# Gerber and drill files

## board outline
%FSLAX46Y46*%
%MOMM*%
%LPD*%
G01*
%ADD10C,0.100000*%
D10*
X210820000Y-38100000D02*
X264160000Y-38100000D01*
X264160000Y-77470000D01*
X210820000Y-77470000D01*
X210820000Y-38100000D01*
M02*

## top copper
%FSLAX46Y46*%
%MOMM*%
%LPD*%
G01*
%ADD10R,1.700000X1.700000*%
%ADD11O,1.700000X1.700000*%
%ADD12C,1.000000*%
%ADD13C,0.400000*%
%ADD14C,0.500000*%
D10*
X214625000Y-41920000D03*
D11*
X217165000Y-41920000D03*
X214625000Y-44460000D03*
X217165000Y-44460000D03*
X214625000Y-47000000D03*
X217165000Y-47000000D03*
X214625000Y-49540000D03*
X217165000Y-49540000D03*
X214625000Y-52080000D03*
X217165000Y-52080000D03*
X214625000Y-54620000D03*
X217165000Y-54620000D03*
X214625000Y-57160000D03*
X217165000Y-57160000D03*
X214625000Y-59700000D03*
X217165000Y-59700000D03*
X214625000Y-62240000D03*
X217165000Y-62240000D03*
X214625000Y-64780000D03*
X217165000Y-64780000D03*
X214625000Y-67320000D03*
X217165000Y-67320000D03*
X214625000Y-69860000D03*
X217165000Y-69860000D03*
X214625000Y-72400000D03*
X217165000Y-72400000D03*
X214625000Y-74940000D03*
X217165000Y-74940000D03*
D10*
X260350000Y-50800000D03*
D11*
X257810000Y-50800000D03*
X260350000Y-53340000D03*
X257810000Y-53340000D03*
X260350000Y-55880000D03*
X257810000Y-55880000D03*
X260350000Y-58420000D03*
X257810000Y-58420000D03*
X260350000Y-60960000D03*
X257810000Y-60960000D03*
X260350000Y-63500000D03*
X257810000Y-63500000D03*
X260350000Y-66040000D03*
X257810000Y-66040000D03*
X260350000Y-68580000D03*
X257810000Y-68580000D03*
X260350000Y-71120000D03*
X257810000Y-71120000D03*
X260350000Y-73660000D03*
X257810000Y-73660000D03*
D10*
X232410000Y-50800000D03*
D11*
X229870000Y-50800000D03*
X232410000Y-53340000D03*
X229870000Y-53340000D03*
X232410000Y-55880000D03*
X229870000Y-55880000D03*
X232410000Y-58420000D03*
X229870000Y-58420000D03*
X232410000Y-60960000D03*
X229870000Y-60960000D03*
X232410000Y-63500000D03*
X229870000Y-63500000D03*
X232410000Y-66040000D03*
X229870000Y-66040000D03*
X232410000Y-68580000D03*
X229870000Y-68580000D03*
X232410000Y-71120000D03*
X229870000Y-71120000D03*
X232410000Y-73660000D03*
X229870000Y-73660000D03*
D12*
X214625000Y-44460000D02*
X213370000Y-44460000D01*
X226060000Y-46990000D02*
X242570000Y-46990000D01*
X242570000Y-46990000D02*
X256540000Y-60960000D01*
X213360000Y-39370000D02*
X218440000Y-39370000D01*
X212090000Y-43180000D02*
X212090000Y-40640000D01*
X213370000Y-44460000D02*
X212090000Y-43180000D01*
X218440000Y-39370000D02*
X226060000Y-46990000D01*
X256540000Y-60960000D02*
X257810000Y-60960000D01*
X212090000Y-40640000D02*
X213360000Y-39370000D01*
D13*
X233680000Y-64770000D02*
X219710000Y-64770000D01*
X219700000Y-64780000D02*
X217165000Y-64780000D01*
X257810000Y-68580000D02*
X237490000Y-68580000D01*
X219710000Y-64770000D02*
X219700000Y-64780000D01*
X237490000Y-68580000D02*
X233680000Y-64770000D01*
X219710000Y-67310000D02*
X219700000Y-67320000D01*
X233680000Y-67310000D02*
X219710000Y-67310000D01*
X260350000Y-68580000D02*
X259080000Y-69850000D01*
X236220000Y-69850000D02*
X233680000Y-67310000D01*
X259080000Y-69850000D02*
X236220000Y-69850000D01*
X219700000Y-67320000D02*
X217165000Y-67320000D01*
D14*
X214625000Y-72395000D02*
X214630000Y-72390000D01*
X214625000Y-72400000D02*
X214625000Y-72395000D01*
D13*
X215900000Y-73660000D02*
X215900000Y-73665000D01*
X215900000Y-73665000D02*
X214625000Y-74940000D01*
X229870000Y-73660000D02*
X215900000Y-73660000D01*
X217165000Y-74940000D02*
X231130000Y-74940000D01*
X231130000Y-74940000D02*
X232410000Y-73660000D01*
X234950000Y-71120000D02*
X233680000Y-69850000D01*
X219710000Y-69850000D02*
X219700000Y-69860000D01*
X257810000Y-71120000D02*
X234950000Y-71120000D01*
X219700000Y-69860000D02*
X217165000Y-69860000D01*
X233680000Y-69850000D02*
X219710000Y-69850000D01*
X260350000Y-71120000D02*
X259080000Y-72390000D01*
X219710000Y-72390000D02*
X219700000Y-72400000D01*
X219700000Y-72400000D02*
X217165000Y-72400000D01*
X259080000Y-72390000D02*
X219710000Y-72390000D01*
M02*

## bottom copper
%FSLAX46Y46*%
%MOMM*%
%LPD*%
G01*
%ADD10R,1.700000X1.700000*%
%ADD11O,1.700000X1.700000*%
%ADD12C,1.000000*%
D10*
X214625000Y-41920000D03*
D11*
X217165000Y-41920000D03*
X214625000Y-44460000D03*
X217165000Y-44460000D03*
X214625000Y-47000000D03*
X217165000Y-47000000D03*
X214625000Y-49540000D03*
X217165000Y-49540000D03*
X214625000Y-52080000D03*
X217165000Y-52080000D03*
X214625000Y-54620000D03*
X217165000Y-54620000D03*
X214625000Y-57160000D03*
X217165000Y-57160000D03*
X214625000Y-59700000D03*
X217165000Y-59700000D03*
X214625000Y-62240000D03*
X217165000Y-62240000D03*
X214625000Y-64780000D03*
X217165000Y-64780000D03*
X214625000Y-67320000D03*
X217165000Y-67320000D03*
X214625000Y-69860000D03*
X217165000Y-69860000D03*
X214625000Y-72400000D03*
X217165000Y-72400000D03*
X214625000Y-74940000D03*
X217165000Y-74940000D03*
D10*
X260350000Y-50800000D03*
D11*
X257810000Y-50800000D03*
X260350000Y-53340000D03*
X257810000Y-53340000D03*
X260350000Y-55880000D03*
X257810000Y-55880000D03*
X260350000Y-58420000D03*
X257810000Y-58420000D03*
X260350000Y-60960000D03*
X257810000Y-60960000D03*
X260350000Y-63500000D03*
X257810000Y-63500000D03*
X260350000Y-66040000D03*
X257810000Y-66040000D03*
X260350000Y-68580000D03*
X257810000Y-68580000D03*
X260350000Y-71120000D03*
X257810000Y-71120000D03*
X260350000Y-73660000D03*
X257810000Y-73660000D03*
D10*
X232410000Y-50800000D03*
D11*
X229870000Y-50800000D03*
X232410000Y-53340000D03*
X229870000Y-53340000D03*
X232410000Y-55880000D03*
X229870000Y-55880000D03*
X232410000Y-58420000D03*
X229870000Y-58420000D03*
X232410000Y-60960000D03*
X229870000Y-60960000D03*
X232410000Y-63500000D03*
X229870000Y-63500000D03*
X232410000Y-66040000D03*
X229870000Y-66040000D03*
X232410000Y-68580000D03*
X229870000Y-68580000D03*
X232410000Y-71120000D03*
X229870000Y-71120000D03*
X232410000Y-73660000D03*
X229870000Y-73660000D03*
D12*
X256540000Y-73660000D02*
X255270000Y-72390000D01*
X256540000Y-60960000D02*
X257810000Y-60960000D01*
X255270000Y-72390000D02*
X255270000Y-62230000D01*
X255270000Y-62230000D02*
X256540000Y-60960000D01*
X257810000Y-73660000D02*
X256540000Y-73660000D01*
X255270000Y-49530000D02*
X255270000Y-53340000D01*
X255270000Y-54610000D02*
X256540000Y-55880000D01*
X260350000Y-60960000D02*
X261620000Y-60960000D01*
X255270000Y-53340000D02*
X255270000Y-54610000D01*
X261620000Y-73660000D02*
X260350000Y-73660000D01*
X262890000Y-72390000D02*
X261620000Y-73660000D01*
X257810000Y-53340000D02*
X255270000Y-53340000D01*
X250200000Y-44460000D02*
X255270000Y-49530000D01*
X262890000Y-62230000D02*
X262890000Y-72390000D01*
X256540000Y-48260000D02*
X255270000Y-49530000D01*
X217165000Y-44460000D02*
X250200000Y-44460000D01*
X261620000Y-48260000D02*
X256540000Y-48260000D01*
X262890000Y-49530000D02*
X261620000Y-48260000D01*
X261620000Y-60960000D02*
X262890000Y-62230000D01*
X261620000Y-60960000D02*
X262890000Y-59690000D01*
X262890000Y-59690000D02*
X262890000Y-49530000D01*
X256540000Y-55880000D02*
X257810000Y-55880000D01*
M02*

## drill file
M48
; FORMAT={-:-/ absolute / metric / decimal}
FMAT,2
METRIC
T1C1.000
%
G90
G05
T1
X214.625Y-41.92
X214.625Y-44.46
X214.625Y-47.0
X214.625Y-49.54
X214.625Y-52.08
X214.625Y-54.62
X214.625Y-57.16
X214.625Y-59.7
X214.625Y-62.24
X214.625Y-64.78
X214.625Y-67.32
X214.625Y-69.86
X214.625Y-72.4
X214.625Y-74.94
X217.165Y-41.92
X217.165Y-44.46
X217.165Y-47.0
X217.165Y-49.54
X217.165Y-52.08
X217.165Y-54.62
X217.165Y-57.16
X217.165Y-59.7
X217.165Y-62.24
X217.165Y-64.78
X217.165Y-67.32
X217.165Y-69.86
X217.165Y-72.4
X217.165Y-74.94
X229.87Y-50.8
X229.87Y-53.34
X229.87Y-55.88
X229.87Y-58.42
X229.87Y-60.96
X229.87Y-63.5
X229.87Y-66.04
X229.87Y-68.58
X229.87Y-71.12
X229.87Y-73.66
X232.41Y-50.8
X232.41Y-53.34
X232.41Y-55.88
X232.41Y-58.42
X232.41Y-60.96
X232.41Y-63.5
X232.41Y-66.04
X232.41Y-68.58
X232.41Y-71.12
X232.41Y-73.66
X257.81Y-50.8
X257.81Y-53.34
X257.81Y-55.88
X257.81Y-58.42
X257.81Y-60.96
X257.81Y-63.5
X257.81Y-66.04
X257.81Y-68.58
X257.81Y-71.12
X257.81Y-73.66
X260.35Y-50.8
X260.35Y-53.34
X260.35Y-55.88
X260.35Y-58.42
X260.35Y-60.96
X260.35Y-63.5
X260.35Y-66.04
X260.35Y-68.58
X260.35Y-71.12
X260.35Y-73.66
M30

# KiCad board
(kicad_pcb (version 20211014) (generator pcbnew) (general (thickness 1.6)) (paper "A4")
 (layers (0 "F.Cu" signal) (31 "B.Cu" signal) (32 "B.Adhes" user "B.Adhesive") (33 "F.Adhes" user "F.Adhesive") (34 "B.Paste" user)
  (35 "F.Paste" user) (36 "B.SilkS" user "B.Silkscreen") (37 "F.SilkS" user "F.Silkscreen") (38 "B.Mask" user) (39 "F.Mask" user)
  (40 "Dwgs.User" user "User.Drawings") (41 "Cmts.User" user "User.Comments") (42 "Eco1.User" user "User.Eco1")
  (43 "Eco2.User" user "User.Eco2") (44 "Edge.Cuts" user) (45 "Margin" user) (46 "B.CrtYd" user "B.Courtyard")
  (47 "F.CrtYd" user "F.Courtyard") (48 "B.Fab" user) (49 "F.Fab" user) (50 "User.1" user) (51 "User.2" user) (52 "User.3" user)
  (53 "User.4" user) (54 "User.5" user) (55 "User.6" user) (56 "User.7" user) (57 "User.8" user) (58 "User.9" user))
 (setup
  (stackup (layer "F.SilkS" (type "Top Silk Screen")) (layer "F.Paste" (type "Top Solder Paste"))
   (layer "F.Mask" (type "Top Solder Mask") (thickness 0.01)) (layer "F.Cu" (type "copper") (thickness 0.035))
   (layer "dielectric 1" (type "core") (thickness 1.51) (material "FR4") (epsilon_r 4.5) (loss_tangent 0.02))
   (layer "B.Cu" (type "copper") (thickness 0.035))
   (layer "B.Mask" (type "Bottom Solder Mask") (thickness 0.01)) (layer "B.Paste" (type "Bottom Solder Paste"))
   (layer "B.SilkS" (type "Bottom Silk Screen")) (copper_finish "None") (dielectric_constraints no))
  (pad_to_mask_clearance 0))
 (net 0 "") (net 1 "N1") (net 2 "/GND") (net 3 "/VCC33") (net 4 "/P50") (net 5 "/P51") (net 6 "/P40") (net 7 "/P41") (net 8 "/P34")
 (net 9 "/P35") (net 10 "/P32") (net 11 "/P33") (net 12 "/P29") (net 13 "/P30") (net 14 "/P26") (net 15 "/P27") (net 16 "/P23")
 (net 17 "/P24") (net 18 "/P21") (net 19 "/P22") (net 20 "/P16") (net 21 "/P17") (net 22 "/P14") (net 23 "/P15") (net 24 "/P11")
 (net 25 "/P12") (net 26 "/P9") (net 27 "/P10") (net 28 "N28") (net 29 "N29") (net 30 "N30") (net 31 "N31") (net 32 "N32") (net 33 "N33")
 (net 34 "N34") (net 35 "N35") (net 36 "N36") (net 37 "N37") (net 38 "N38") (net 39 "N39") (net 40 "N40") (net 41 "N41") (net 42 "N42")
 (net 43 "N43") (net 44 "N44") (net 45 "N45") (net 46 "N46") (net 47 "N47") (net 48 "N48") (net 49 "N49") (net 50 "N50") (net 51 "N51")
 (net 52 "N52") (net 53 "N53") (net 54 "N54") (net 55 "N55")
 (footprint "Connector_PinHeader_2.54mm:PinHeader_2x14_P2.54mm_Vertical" (layer "F.Cu") (at 214.625 41.92)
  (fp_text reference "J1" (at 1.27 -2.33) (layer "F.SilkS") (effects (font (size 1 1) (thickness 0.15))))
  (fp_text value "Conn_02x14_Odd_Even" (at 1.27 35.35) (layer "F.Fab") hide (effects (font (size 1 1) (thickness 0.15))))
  (pad "1" thru_hole rect locked (at 0 0) (size 1.7 1.7) (drill 1) (layers *.Cu *.Mask) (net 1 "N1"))
  (pad "2" thru_hole oval locked (at 2.54 0) (size 1.7 1.7) (drill 1) (layers *.Cu *.Mask) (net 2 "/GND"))
  (pad "3" thru_hole oval locked (at 0 2.54) (size 1.7 1.7) (drill 1) (layers *.Cu *.Mask) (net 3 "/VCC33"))
  (pad "4" thru_hole oval locked (at 2.54 2.54) (size 1.7 1.7) (drill 1) (layers *.Cu *.Mask) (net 2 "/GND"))
  (pad "5" thru_hole oval locked (at 0 5.08) (size 1.7 1.7) (drill 1) (layers *.Cu *.Mask) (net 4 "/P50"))
  (pad "6" thru_hole oval locked (at 2.54 5.08) (size 1.7 1.7) (drill 1) (layers *.Cu *.Mask) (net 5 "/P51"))
  (pad "7" thru_hole oval locked (at 0 7.62) (size 1.7 1.7) (drill 1) (layers *.Cu *.Mask) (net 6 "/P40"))
  (pad "8" thru_hole oval locked (at 2.54 7.62) (size 1.7 1.7) (drill 1) (layers *.Cu *.Mask) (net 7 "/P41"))
  (pad "9" thru_hole oval locked (at 0 10.16) (size 1.7 1.7) (drill 1) (layers *.Cu *.Mask) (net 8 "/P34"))
  (pad "10" thru_hole oval locked (at 2.54 10.16) (size 1.7 1.7) (drill 1) (layers *.Cu *.Mask) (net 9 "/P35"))
  (pad "11" thru_hole oval locked (at 0 12.7) (size 1.7 1.7) (drill 1) (layers *.Cu *.Mask) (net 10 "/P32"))
  (pad "12" thru_hole oval locked (at 2.54 12.7) (size 1.7 1.7) (drill 1) (layers *.Cu *.Mask) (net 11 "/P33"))
  (pad "13" thru_hole oval locked (at 0 15.24) (size 1.7 1.7) (drill 1) (layers *.Cu *.Mask) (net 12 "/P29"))
  (pad "14" thru_hole oval locked (at 2.54 15.24) (size 1.7 1.7) (drill 1) (layers *.Cu *.Mask) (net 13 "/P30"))
  (pad "15" thru_hole oval locked (at 0 17.78) (size 1.7 1.7) (drill 1) (layers *.Cu *.Mask) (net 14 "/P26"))
  (pad "16" thru_hole oval locked (at 2.54 17.78) (size 1.7 1.7) (drill 1) (layers *.Cu *.Mask) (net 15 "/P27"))
  (pad "17" thru_hole oval locked (at 0 20.32) (size 1.7 1.7) (drill 1) (layers *.Cu *.Mask) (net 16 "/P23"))
  (pad "18" thru_hole oval locked (at 2.54 20.32) (size 1.7 1.7) (drill 1) (layers *.Cu *.Mask) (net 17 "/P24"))
  (pad "19" thru_hole oval locked (at 0 22.86) (size 1.7 1.7) (drill 1) (layers *.Cu *.Mask) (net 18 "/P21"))
  (pad "20" thru_hole oval locked (at 2.54 22.86) (size 1.7 1.7) (drill 1) (layers *.Cu *.Mask) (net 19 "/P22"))
  (pad "21" thru_hole oval locked (at 0 25.4) (size 1.7 1.7) (drill 1) (layers *.Cu *.Mask) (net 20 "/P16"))
  (pad "22" thru_hole oval locked (at 2.54 25.4) (size 1.7 1.7) (drill 1) (layers *.Cu *.Mask) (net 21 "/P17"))
  (pad "23" thru_hole oval locked (at 0 27.94) (size 1.7 1.7) (drill 1) (layers *.Cu *.Mask) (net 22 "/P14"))
  (pad "24" thru_hole oval locked (at 2.54 27.94) (size 1.7 1.7) (drill 1) (layers *.Cu *.Mask) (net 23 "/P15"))
  (pad "25" thru_hole oval locked (at 0 30.48) (size 1.7 1.7) (drill 1) (layers *.Cu *.Mask) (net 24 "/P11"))
  (pad "26" thru_hole oval locked (at 2.54 30.48) (size 1.7 1.7) (drill 1) (layers *.Cu *.Mask) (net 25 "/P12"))
  (pad "27" thru_hole oval locked (at 0 33.02) (size 1.7 1.7) (drill 1) (layers *.Cu *.Mask) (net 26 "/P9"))
  (pad "28" thru_hole oval locked (at 2.54 33.02) (size 1.7 1.7) (drill 1) (layers *.Cu *.Mask) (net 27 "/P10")))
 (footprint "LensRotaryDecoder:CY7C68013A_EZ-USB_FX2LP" (layer "B.Cu") (at 248.38 62.225 180)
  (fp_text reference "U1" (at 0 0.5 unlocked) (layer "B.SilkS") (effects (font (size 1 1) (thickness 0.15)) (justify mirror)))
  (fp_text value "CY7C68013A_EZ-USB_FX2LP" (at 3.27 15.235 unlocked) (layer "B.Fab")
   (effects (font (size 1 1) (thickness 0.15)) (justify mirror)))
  (pad "1" thru_hole rect (at -11.97 11.425 180) (size 1.7 1.7) (drill 1) (layers *.Cu *.Mask) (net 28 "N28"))
  (pad "2" thru_hole oval (at -9.43 11.425 180) (size 1.7 1.7) (drill 1) (layers *.Cu *.Mask) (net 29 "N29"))
  (pad "3" thru_hole oval (at -11.97 8.885 180) (size 1.7 1.7) (drill 1) (layers *.Cu *.Mask) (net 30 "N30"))
  (pad "4" thru_hole oval (at -9.43 8.885 180) (size 1.7 1.7) (drill 1) (layers *.Cu *.Mask) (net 2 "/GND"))
  (pad "5" thru_hole oval (at -11.97 6.345 180) (size 1.7 1.7) (drill 1) (layers *.Cu *.Mask) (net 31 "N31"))
  (pad "6" thru_hole oval (at -9.43 6.345 180) (size 1.7 1.7) (drill 1) (layers *.Cu *.Mask) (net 2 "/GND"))
  (pad "7" thru_hole oval (at -11.97 3.805 180) (size 1.7 1.7) (drill 1) (layers *.Cu *.Mask) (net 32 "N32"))
  (pad "8" thru_hole oval (at -9.43 3.805 180) (size 1.7 1.7) (drill 1) (layers *.Cu *.Mask) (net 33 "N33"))
  (pad "9" thru_hole oval (at -11.97 1.265 180) (size 1.7 1.7) (drill 1) (layers *.Cu *.Mask) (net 2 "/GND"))
  (pad "10" thru_hole oval (at -9.43 1.265 180) (size 1.7 1.7) (drill 1) (layers *.Cu *.Mask) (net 3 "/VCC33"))
  (pad "11" thru_hole oval (at -11.97 -1.275 180) (size 1.7 1.7) (drill 1) (layers *.Cu *.Mask) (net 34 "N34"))
  (pad "12" thru_hole oval (at -9.43 -1.275 180) (size 1.7 1.7) (drill 1) (layers *.Cu *.Mask) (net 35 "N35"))
  (pad "13" thru_hole oval (at -11.97 -3.815 180) (size 1.7 1.7) (drill 1) (layers *.Cu *.Mask) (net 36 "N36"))
  (pad "14" thru_hole oval (at -9.43 -3.815 180) (size 1.7 1.7) (drill 1) (layers *.Cu *.Mask) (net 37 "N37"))
  (pad "15" thru_hole oval (at -11.97 -6.355 180) (size 1.7 1.7) (drill 1) (layers *.Cu *.Mask) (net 21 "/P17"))
  (pad "16" thru_hole oval (at -9.43 -6.355 180) (size 1.7 1.7) (drill 1) (layers *.Cu *.Mask) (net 19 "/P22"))
  (pad "17" thru_hole oval (at -11.97 -8.895 180) (size 1.7 1.7) (drill 1) (layers *.Cu *.Mask) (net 25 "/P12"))
  (pad "18" thru_hole oval (at -9.43 -8.895 180) (size 1.7 1.7) (drill 1) (layers *.Cu *.Mask) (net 23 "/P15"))
  (pad "19" thru_hole oval (at -11.97 -11.435 180) (size 1.7 1.7) (drill 1) (layers *.Cu *.Mask) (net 2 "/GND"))
  (pad "20" thru_hole oval (at -9.43 -11.435 180) (size 1.7 1.7) (drill 1) (layers *.Cu *.Mask) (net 3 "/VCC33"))
  (pad "21" thru_hole rect (at 15.97 11.425 180) (size 1.7 1.7) (drill 1) (layers *.Cu *.Mask) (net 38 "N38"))
  (pad "22" thru_hole oval (at 18.51 11.425 180) (size 1.7 1.7) (drill 1) (layers *.Cu *.Mask) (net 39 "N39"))
  (pad "23" thru_hole oval (at 15.97 8.885 180) (size 1.7 1.7) (drill 1) (layers *.Cu *.Mask) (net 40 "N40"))
  (pad "24" thru_hole oval (at 18.51 8.885 180) (size 1.7 1.7) (drill 1) (layers *.Cu *.Mask) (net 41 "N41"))
  (pad "25" thru_hole oval (at 15.97 6.345 180) (size 1.7 1.7) (drill 1) (layers *.Cu *.Mask) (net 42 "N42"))
  (pad "26" thru_hole oval (at 18.51 6.345 180) (size 1.7 1.7) (drill 1) (layers *.Cu *.Mask) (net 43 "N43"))
  (pad "27" thru_hole oval (at 15.97 3.805 180) (size 1.7 1.7) (drill 1) (layers *.Cu *.Mask) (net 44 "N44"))
  (pad "28" thru_hole oval (at 18.51 3.805 180) (size 1.7 1.7) (drill 1) (layers *.Cu *.Mask) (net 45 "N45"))
  (pad "29" thru_hole oval (at 15.97 1.265 180) (size 1.7 1.7) (drill 1) (layers *.Cu *.Mask) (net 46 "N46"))
  (pad "30" thru_hole oval (at 18.51 1.265 180) (size 1.7 1.7) (drill 1) (layers *.Cu *.Mask) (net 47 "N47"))
  (pad "31" thru_hole oval (at 15.97 -1.275 180) (size 1.7 1.7) (drill 1) (layers *.Cu *.Mask) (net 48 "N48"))
  (pad "32" thru_hole oval (at 18.51 -1.275 180) (size 1.7 1.7) (drill 1) (layers *.Cu *.Mask) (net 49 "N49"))
  (pad "33" thru_hole oval (at 15.97 -3.815 180) (size 1.7 1.7) (drill 1) (layers *.Cu *.Mask) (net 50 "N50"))
  (pad "34" thru_hole oval (at 18.51 -3.815 180) (size 1.7 1.7) (drill 1) (layers *.Cu *.Mask) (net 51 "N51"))
  (pad "35" thru_hole oval (at 15.97 -6.355 180) (size 1.7 1.7) (drill 1) (layers *.Cu *.Mask) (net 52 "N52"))
  (pad "36" thru_hole oval (at 18.51 -6.355 180) (size 1.7 1.7) (drill 1) (layers *.Cu *.Mask) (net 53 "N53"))
  (pad "37" thru_hole oval (at 15.97 -8.895 180) (size 1.7 1.7) (drill 1) (layers *.Cu *.Mask) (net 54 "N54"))
  (pad "38" thru_hole oval (at 18.51 -8.895 180) (size 1.7 1.7) (drill 1) (layers *.Cu *.Mask) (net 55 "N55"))
  (pad "39" thru_hole oval (at 15.97 -11.435 180) (size 1.7 1.7) (drill 1) (layers *.Cu *.Mask) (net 27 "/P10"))
  (pad "40" thru_hole oval (at 18.51 -11.435 180) (size 1.7 1.7) (drill 1) (layers *.Cu *.Mask) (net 26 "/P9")))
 (gr_rect (start 210.82 38.1) (end 264.16 77.47) (layer "Edge.Cuts") (width 0.1) (fill none))
 (segment (start 214.625 44.46) (end 213.37 44.46) (width 1) (layer "F.Cu") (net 3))
 (segment (start 226.06 46.99) (end 242.57 46.99) (width 1) (layer "F.Cu") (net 3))
 (segment (start 242.57 46.99) (end 256.54 60.96) (width 1) (layer "F.Cu") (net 3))
 (segment (start 213.36 39.37) (end 218.44 39.37) (width 1) (layer "F.Cu") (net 3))
 (segment (start 212.09 43.18) (end 212.09 40.64) (width 1) (layer "F.Cu") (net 3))
 (segment (start 213.37 44.46) (end 212.09 43.18) (width 1) (layer "F.Cu") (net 3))
 (segment (start 218.44 39.37) (end 226.06 46.99) (width 1) (layer "F.Cu") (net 3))
 (segment (start 256.54 60.96) (end 257.81 60.96) (width 1) (layer "F.Cu") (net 3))
 (segment (start 212.09 40.64) (end 213.36 39.37) (width 1) (layer "F.Cu") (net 3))
 (segment (start 256.54 73.66) (end 255.27 72.39) (width 1) (layer "B.Cu") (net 3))
 (segment (start 256.54 60.96) (end 257.81 60.96) (width 1) (layer "B.Cu") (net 3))
 (segment (start 255.27 72.39) (end 255.27 62.23) (width 1) (layer "B.Cu") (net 3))
 (segment (start 255.27 62.23) (end 256.54 60.96) (width 1) (layer "B.Cu") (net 3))
 (segment (start 257.81 73.66) (end 256.54 73.66) (width 1) (layer "B.Cu") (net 3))
 (segment (start 255.27 49.53) (end 255.27 53.34) (width 1) (layer "B.Cu") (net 2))
 (segment (start 255.27 54.61) (end 256.54 55.88) (width 1) (layer "B.Cu") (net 2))
 (segment (start 260.35 60.96) (end 261.62 60.96) (width 1) (layer "B.Cu") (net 2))
 (segment (start 255.27 53.34) (end 255.27 54.61) (width 1) (layer "B.Cu") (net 2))
 (segment (start 261.62 73.66) (end 260.35 73.66) (width 1) (layer "B.Cu") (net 2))
 (segment (start 262.89 72.39) (end 261.62 73.66) (width 1) (layer "B.Cu") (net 2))
 (segment (start 257.81 53.34) (end 255.27 53.34) (width 1) (layer "B.Cu") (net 2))
 (segment (start 250.2 44.46) (end 255.27 49.53) (width 1) (layer "B.Cu") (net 2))
 (segment (start 262.89 62.23) (end 262.89 72.39) (width 1) (layer "B.Cu") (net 2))
 (segment (start 256.54 48.26) (end 255.27 49.53) (width 1) (layer "B.Cu") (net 2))
 (segment (start 217.165 44.46) (end 250.2 44.46) (width 1) (layer "B.Cu") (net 2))
 (segment (start 261.62 48.26) (end 256.54 48.26) (width 1) (layer "B.Cu") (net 2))
 (segment (start 262.89 49.53) (end 261.62 48.26) (width 1) (layer "B.Cu") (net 2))
 (segment (start 261.62 60.96) (end 262.89 62.23) (width 1) (layer "B.Cu") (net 2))
 (segment (start 261.62 60.96) (end 262.89 59.69) (width 1) (layer "B.Cu") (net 2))
 (segment (start 262.89 59.69) (end 262.89 49.53) (width 1) (layer "B.Cu") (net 2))
 (segment (start 256.54 55.88) (end 257.81 55.88) (width 1) (layer "B.Cu") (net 2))
 (segment (start 233.68 64.77) (end 219.71 64.77) (width 0.4) (layer "F.Cu") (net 19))
 (segment (start 219.7 64.78) (end 217.165 64.78) (width 0.4) (layer "F.Cu") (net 19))
 (segment (start 257.81 68.58) (end 237.49 68.58) (width 0.4) (layer "F.Cu") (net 19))
 (segment (start 219.71 64.77) (end 219.7 64.78) (width 0.4) (layer "F.Cu") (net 19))
 (segment (start 237.49 68.58) (end 233.68 64.77) (width 0.4) (layer "F.Cu") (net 19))
 (segment (start 219.71 67.31) (end 219.7 67.32) (width 0.4) (layer "F.Cu") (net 21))
 (segment (start 233.68 67.31) (end 219.71 67.31) (width 0.4) (layer "F.Cu") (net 21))
 (segment (start 260.35 68.58) (end 259.08 69.85) (width 0.4) (layer "F.Cu") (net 21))
 (segment (start 236.22 69.85) (end 233.68 67.31) (width 0.4) (layer "F.Cu") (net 21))
 (segment (start 259.08 69.85) (end 236.22 69.85) (width 0.4) (layer "F.Cu") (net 21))
 (segment (start 219.7 67.32) (end 217.165 67.32) (width 0.4) (layer "F.Cu") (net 21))
 (segment (start 214.625 72.395) (end 214.63 72.39) (width 0.5) (layer "F.Cu") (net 24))
 (segment (start 214.625 72.4) (end 214.625 72.395) (width 0.5) (layer "F.Cu") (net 24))
 (segment (start 215.9 73.66) (end 215.9 73.665) (width 0.4) (layer "F.Cu") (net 26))
 (segment (start 215.9 73.665) (end 214.625 74.94) (width 0.4) (layer "F.Cu") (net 26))
 (segment (start 229.87 73.66) (end 215.9 73.66) (width 0.4) (layer "F.Cu") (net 26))
 (segment (start 217.165 74.94) (end 231.13 74.94) (width 0.4) (layer "F.Cu") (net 27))
 (segment (start 231.13 74.94) (end 232.41 73.66) (width 0.4) (layer "F.Cu") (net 27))
 (segment (start 234.95 71.12) (end 233.68 69.85) (width 0.4) (layer "F.Cu") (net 23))
 (segment (start 219.71 69.85) (end 219.7 69.86) (width 0.4) (layer "F.Cu") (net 23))
 (segment (start 257.81 71.12) (end 234.95 71.12) (width 0.4) (layer "F.Cu") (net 23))
 (segment (start 219.7 69.86) (end 217.165 69.86) (width 0.4) (layer "F.Cu") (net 23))
 (segment (start 233.68 69.85) (end 219.71 69.85) (width 0.4) (layer "F.Cu") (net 23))
 (segment (start 260.35 71.12) (end 259.08 72.39) (width 0.4) (layer "F.Cu") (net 25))
 (segment (start 219.71 72.39) (end 219.7 72.4) (width 0.4) (layer "F.Cu") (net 25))
 (segment (start 219.7 72.4) (end 217.165 72.4) (width 0.4) (layer "F.Cu") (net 25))
 (segment (start 259.08 72.39) (end 219.71 72.39) (width 0.4) (layer "F.Cu") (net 25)))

